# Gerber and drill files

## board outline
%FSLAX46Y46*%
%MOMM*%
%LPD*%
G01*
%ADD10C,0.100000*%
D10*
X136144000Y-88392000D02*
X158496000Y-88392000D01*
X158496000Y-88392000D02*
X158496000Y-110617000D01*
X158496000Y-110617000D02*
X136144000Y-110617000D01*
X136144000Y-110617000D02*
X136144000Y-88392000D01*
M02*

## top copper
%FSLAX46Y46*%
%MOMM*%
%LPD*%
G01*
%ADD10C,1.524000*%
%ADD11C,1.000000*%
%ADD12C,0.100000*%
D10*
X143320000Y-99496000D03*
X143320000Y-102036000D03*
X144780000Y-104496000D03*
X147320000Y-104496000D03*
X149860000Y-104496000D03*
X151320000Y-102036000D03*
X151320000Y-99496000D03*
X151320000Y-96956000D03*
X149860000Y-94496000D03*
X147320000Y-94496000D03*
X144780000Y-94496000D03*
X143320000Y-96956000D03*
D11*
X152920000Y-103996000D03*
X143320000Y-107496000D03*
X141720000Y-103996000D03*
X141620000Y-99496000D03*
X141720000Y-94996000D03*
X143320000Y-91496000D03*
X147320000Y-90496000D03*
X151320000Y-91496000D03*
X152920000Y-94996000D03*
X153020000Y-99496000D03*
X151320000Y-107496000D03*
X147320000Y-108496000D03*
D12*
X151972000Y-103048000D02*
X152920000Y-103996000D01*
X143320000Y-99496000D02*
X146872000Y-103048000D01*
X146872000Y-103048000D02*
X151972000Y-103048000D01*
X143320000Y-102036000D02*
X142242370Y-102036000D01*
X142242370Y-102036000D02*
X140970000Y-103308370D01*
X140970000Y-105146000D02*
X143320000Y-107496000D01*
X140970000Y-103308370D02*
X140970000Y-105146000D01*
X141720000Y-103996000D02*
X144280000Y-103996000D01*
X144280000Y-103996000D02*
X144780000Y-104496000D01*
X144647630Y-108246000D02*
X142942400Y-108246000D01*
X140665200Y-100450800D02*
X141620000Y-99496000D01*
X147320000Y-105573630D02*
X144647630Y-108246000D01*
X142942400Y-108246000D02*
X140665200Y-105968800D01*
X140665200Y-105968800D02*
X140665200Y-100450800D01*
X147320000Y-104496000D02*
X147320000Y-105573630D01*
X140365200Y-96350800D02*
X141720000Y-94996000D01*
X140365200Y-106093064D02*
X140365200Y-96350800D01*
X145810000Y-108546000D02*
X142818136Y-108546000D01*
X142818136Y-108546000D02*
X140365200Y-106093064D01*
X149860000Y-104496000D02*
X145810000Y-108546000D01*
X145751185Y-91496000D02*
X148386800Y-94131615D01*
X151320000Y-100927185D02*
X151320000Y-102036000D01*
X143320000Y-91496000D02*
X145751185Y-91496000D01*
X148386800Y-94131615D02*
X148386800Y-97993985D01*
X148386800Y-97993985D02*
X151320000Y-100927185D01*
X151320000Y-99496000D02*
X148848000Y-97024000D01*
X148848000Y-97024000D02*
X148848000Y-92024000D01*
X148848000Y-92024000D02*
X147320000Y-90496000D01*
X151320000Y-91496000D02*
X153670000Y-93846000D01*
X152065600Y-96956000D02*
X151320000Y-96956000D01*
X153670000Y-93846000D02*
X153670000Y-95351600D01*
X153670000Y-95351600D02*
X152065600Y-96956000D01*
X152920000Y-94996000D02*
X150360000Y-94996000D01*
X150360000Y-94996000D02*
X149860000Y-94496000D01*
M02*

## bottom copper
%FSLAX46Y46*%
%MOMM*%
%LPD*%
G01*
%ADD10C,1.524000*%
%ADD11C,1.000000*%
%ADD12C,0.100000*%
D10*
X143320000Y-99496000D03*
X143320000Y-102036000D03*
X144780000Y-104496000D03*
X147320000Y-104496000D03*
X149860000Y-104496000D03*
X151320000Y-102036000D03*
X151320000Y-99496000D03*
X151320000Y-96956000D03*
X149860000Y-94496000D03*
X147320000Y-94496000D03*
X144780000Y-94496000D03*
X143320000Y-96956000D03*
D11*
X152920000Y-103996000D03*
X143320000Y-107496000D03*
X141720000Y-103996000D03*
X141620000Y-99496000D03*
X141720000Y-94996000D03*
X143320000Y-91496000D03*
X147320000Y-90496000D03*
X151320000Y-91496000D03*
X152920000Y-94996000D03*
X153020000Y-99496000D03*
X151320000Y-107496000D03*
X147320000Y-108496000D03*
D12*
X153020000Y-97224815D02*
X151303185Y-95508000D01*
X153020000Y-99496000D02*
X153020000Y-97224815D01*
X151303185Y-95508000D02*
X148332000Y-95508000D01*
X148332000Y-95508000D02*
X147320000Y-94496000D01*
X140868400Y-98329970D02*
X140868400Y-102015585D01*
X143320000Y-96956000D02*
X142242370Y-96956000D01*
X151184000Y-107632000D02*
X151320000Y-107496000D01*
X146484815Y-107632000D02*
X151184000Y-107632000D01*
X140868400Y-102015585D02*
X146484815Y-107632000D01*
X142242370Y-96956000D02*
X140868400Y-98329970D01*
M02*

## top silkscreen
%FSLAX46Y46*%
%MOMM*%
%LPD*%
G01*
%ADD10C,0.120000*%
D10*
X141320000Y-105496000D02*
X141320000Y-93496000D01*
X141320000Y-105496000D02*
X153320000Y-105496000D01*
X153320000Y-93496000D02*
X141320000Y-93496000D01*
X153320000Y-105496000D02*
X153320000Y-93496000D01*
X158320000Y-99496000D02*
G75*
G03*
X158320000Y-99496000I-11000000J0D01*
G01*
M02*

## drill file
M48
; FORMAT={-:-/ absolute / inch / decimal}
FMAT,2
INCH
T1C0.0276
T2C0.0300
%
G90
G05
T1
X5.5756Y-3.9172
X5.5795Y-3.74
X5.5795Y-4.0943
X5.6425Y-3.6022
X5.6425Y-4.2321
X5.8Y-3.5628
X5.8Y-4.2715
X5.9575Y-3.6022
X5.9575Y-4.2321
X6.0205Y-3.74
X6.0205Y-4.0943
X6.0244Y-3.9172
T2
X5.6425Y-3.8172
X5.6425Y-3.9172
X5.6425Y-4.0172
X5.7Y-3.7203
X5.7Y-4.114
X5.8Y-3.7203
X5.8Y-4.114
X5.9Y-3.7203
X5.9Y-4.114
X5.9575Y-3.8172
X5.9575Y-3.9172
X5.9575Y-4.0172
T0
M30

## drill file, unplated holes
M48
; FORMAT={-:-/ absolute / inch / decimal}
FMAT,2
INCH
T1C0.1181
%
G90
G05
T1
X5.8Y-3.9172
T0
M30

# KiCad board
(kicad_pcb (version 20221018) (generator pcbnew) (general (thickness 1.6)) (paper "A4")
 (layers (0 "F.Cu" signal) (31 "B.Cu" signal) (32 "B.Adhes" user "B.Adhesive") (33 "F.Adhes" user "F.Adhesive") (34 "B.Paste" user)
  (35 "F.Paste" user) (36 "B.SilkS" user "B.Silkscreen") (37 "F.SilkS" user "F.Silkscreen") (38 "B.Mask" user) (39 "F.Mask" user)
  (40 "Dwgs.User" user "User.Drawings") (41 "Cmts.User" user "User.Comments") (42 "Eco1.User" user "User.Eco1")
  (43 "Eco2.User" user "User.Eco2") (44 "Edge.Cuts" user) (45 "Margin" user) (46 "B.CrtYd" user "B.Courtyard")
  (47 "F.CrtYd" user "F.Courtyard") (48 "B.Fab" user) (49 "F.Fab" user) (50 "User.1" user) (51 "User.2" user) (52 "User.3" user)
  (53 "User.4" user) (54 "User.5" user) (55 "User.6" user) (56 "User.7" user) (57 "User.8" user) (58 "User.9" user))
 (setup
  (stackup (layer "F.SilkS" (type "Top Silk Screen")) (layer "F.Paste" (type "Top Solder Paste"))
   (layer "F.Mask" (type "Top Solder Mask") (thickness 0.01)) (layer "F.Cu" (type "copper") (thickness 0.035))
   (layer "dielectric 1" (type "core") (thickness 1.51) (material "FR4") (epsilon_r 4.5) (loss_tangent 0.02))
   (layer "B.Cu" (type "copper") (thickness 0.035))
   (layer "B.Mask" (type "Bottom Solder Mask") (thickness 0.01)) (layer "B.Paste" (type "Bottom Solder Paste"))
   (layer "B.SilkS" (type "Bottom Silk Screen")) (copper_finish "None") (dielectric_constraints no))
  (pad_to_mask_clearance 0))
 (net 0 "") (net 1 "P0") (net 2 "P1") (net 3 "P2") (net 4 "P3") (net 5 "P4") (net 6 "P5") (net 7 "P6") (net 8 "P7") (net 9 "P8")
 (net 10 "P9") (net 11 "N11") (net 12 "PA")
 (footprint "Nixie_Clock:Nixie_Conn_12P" (layer "F.Cu") (at 147.32 99.496)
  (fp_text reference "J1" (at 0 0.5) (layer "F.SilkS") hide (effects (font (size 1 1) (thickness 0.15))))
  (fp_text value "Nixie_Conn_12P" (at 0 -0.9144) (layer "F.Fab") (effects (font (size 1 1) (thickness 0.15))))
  (fp_line (start -6 6) (end -6 -6) (stroke (width 0.12) (type solid)) (layer "F.SilkS"))
  (fp_line (start -6 6) (end 6 6) (stroke (width 0.12) (type solid)) (layer "F.SilkS"))
  (fp_line (start 6 -6) (end -6 -6) (stroke (width 0.12) (type solid)) (layer "F.SilkS"))
  (fp_line (start 6 6) (end 6 -6) (stroke (width 0.12) (type solid)) (layer "F.SilkS"))
  (pad "0" thru_hole circle (at -4 0) (size 1.524 1.524) (drill 0.762) (layers "*.Cu" "*.Mask") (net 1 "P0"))
  (pad "1" thru_hole circle (at -4 2.54) (size 1.524 1.524) (drill 0.762) (layers "*.Cu" "*.Mask") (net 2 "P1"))
  (pad "2" thru_hole circle (at -2.54 5) (size 1.524 1.524) (drill 0.762) (layers "*.Cu" "*.Mask") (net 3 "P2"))
  (pad "3" thru_hole circle (at 0 5) (size 1.524 1.524) (drill 0.762) (layers "*.Cu" "*.Mask") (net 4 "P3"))
  (pad "4" thru_hole circle (at 2.54 5) (size 1.524 1.524) (drill 0.762) (layers "*.Cu" "*.Mask") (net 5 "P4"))
  (pad "5" thru_hole circle (at 4 2.54) (size 1.524 1.524) (drill 0.762) (layers "*.Cu" "*.Mask") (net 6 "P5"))
  (pad "6" thru_hole circle (at 4 0) (size 1.524 1.524) (drill 0.762) (layers "*.Cu" "*.Mask") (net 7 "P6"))
  (pad "7" thru_hole circle (at 4 -2.54) (size 1.524 1.524) (drill 0.762) (layers "*.Cu" "*.Mask") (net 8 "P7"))
  (pad "8" thru_hole circle (at 2.54 -5) (size 1.524 1.524) (drill 0.762) (layers "*.Cu" "*.Mask") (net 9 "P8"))
  (pad "9" thru_hole circle (at 0 -5) (size 1.524 1.524) (drill 0.762) (layers "*.Cu" "*.Mask") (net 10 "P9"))
  (pad "10" thru_hole circle (at -2.54 -5) (size 1.524 1.524) (drill 0.762) (layers "*.Cu" "*.Mask") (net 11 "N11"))
  (pad "A" thru_hole circle (at -4 -2.54) (size 1.524 1.524) (drill 0.762) (layers "*.Cu" "*.Mask") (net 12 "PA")))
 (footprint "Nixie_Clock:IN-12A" (layer "F.Cu") (at 147.32 99.496)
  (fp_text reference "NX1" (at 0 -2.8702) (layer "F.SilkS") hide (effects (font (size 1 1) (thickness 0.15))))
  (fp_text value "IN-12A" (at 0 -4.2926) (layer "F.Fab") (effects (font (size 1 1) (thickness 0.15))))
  (fp_circle (center 0 0) (end 11 0) (stroke (width 0.12) (type solid)) (fill none) (layer "F.SilkS"))
  (pad "" np_thru_hole circle (at 0 0) (size 3 3) (drill 3) (layers "*.Cu" "*.Mask"))
  (pad "0" thru_hole circle (at 5.6 4.5) (size 1 1) (drill 0.7) (layers "*.Cu" "*.Mask") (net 1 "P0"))
  (pad "1" thru_hole circle (at -4 8) (size 1 1) (drill 0.7) (layers "*.Cu" "*.Mask") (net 2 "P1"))
  (pad "2" thru_hole circle (at -5.6 4.5) (size 1 1) (drill 0.7) (layers "*.Cu" "*.Mask") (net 3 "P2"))
  (pad "3" thru_hole circle (at -5.7 0) (size 1 1) (drill 0.7) (layers "*.Cu" "*.Mask") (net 4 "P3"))
  (pad "4" thru_hole circle (at -5.6 -4.5) (size 1 1) (drill 0.7) (layers "*.Cu" "*.Mask") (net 5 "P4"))
  (pad "5" thru_hole circle (at -4 -8) (size 1 1) (drill 0.7) (layers "*.Cu" "*.Mask") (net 6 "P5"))
  (pad "6" thru_hole circle (at 0 -9) (size 1 1) (drill 0.7) (layers "*.Cu" "*.Mask") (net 7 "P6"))
  (pad "7" thru_hole circle (at 4 -8) (size 1 1) (drill 0.7) (layers "*.Cu" "*.Mask") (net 8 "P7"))
  (pad "8" thru_hole circle (at 5.6 -4.5) (size 1 1) (drill 0.7) (layers "*.Cu" "*.Mask") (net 9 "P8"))
  (pad "9" thru_hole circle (at 5.7 0) (size 1 1) (drill 0.7) (layers "*.Cu" "*.Mask") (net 10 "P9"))
  (pad "A" thru_hole circle (at 4 8) (size 1 1) (drill 0.7) (layers "*.Cu" "*.Mask") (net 12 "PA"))
  (pad "DP" thru_hole circle (at 0 9) (size 1 1) (drill 0.7) (layers "*.Cu" "*.Mask")))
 (gr_rect (start 136.144 88.392) (end 158.496 110.617) (stroke (width 0.1) (type default)) (fill none) (layer "Edge.Cuts"))
 (segment (start 151.972 103.048) (end 152.92 103.996) (width 0.1) (layer "F.Cu") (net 1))
 (segment (start 143.32 99.496) (end 146.872 103.048) (width 0.1) (layer "F.Cu") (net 1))
 (segment (start 146.872 103.048) (end 151.972 103.048) (width 0.1) (layer "F.Cu") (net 1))
 (segment (start 143.32 102.036) (end 142.24237 102.036) (width 0.1) (layer "F.Cu") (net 2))
 (segment (start 142.24237 102.036) (end 140.97 103.30837) (width 0.1) (layer "F.Cu") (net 2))
 (segment (start 140.97 105.146) (end 143.32 107.496) (width 0.1) (layer "F.Cu") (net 2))
 (segment (start 140.97 103.30837) (end 140.97 105.146) (width 0.1) (layer "F.Cu") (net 2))
 (segment (start 141.72 103.996) (end 144.28 103.996) (width 0.1) (layer "F.Cu") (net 3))
 (segment (start 144.28 103.996) (end 144.78 104.496) (width 0.1) (layer "F.Cu") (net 3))
 (segment (start 144.64763 108.246) (end 142.9424 108.246) (width 0.1) (layer "F.Cu") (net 4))
 (segment (start 140.6652 100.4508) (end 141.62 99.496) (width 0.1) (layer "F.Cu") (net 4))
 (segment (start 147.32 105.57363) (end 144.64763 108.246) (width 0.1) (layer "F.Cu") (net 4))
 (segment (start 142.9424 108.246) (end 140.6652 105.9688) (width 0.1) (layer "F.Cu") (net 4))
 (segment (start 140.6652 105.9688) (end 140.6652 100.4508) (width 0.1) (layer "F.Cu") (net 4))
 (segment (start 147.32 104.496) (end 147.32 105.57363) (width 0.1) (layer "F.Cu") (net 4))
 (segment (start 140.3652 96.3508) (end 141.72 94.996) (width 0.1) (layer "F.Cu") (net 5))
 (segment (start 140.3652 106.093064) (end 140.3652 96.3508) (width 0.1) (layer "F.Cu") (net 5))
 (segment (start 145.81 108.546) (end 142.818136 108.546) (width 0.1) (layer "F.Cu") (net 5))
 (segment (start 142.818136 108.546) (end 140.3652 106.093064) (width 0.1) (layer "F.Cu") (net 5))
 (segment (start 149.86 104.496) (end 145.81 108.546) (width 0.1) (layer "F.Cu") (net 5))
 (segment (start 145.751185 91.496) (end 148.3868 94.131615) (width 0.1) (layer "F.Cu") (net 6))
 (segment (start 151.32 100.927185) (end 151.32 102.036) (width 0.1) (layer "F.Cu") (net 6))
 (segment (start 143.32 91.496) (end 145.751185 91.496) (width 0.1) (layer "F.Cu") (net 6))
 (segment (start 148.3868 94.131615) (end 148.3868 97.993985) (width 0.1) (layer "F.Cu") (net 6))
 (segment (start 148.3868 97.993985) (end 151.32 100.927185) (width 0.1) (layer "F.Cu") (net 6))
 (segment (start 151.32 99.496) (end 148.848 97.024) (width 0.1) (layer "F.Cu") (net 7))
 (segment (start 148.848 97.024) (end 148.848 92.024) (width 0.1) (layer "F.Cu") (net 7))
 (segment (start 148.848 92.024) (end 147.32 90.496) (width 0.1) (layer "F.Cu") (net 7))
 (segment (start 151.32 91.496) (end 153.67 93.846) (width 0.1) (layer "F.Cu") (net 8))
 (segment (start 152.0656 96.956) (end 151.32 96.956) (width 0.1) (layer "F.Cu") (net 8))
 (segment (start 153.67 93.846) (end 153.67 95.3516) (width 0.1) (layer "F.Cu") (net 8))
 (segment (start 153.67 95.3516) (end 152.0656 96.956) (width 0.1) (layer "F.Cu") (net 8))
 (segment (start 152.92 94.996) (end 150.36 94.996) (width 0.1) (layer "F.Cu") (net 9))
 (segment (start 150.36 94.996) (end 149.86 94.496) (width 0.1) (layer "F.Cu") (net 9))
 (segment (start 153.02 97.224815) (end 151.303185 95.508) (width 0.1) (layer "B.Cu") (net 10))
 (segment (start 153.02 99.496) (end 153.02 97.224815) (width 0.1) (layer "B.Cu") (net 10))
 (segment (start 151.303185 95.508) (end 148.332 95.508) (width 0.1) (layer "B.Cu") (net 10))
 (segment (start 148.332 95.508) (end 147.32 94.496) (width 0.1) (layer "B.Cu") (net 10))
 (segment (start 140.8684 98.32997) (end 140.8684 102.015585) (width 0.1) (layer "B.Cu") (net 12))
 (segment (start 143.32 96.956) (end 142.24237 96.956) (width 0.1) (layer "B.Cu") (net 12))
 (segment (start 151.184 107.632) (end 151.32 107.496) (width 0.1) (layer "B.Cu") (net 12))
 (segment (start 146.484815 107.632) (end 151.184 107.632) (width 0.1) (layer "B.Cu") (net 12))
 (segment (start 140.8684 102.015585) (end 146.484815 107.632) (width 0.1) (layer "B.Cu") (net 12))
 (segment (start 142.24237 96.956) (end 140.8684 98.32997) (width 0.1) (layer "B.Cu") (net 12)))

